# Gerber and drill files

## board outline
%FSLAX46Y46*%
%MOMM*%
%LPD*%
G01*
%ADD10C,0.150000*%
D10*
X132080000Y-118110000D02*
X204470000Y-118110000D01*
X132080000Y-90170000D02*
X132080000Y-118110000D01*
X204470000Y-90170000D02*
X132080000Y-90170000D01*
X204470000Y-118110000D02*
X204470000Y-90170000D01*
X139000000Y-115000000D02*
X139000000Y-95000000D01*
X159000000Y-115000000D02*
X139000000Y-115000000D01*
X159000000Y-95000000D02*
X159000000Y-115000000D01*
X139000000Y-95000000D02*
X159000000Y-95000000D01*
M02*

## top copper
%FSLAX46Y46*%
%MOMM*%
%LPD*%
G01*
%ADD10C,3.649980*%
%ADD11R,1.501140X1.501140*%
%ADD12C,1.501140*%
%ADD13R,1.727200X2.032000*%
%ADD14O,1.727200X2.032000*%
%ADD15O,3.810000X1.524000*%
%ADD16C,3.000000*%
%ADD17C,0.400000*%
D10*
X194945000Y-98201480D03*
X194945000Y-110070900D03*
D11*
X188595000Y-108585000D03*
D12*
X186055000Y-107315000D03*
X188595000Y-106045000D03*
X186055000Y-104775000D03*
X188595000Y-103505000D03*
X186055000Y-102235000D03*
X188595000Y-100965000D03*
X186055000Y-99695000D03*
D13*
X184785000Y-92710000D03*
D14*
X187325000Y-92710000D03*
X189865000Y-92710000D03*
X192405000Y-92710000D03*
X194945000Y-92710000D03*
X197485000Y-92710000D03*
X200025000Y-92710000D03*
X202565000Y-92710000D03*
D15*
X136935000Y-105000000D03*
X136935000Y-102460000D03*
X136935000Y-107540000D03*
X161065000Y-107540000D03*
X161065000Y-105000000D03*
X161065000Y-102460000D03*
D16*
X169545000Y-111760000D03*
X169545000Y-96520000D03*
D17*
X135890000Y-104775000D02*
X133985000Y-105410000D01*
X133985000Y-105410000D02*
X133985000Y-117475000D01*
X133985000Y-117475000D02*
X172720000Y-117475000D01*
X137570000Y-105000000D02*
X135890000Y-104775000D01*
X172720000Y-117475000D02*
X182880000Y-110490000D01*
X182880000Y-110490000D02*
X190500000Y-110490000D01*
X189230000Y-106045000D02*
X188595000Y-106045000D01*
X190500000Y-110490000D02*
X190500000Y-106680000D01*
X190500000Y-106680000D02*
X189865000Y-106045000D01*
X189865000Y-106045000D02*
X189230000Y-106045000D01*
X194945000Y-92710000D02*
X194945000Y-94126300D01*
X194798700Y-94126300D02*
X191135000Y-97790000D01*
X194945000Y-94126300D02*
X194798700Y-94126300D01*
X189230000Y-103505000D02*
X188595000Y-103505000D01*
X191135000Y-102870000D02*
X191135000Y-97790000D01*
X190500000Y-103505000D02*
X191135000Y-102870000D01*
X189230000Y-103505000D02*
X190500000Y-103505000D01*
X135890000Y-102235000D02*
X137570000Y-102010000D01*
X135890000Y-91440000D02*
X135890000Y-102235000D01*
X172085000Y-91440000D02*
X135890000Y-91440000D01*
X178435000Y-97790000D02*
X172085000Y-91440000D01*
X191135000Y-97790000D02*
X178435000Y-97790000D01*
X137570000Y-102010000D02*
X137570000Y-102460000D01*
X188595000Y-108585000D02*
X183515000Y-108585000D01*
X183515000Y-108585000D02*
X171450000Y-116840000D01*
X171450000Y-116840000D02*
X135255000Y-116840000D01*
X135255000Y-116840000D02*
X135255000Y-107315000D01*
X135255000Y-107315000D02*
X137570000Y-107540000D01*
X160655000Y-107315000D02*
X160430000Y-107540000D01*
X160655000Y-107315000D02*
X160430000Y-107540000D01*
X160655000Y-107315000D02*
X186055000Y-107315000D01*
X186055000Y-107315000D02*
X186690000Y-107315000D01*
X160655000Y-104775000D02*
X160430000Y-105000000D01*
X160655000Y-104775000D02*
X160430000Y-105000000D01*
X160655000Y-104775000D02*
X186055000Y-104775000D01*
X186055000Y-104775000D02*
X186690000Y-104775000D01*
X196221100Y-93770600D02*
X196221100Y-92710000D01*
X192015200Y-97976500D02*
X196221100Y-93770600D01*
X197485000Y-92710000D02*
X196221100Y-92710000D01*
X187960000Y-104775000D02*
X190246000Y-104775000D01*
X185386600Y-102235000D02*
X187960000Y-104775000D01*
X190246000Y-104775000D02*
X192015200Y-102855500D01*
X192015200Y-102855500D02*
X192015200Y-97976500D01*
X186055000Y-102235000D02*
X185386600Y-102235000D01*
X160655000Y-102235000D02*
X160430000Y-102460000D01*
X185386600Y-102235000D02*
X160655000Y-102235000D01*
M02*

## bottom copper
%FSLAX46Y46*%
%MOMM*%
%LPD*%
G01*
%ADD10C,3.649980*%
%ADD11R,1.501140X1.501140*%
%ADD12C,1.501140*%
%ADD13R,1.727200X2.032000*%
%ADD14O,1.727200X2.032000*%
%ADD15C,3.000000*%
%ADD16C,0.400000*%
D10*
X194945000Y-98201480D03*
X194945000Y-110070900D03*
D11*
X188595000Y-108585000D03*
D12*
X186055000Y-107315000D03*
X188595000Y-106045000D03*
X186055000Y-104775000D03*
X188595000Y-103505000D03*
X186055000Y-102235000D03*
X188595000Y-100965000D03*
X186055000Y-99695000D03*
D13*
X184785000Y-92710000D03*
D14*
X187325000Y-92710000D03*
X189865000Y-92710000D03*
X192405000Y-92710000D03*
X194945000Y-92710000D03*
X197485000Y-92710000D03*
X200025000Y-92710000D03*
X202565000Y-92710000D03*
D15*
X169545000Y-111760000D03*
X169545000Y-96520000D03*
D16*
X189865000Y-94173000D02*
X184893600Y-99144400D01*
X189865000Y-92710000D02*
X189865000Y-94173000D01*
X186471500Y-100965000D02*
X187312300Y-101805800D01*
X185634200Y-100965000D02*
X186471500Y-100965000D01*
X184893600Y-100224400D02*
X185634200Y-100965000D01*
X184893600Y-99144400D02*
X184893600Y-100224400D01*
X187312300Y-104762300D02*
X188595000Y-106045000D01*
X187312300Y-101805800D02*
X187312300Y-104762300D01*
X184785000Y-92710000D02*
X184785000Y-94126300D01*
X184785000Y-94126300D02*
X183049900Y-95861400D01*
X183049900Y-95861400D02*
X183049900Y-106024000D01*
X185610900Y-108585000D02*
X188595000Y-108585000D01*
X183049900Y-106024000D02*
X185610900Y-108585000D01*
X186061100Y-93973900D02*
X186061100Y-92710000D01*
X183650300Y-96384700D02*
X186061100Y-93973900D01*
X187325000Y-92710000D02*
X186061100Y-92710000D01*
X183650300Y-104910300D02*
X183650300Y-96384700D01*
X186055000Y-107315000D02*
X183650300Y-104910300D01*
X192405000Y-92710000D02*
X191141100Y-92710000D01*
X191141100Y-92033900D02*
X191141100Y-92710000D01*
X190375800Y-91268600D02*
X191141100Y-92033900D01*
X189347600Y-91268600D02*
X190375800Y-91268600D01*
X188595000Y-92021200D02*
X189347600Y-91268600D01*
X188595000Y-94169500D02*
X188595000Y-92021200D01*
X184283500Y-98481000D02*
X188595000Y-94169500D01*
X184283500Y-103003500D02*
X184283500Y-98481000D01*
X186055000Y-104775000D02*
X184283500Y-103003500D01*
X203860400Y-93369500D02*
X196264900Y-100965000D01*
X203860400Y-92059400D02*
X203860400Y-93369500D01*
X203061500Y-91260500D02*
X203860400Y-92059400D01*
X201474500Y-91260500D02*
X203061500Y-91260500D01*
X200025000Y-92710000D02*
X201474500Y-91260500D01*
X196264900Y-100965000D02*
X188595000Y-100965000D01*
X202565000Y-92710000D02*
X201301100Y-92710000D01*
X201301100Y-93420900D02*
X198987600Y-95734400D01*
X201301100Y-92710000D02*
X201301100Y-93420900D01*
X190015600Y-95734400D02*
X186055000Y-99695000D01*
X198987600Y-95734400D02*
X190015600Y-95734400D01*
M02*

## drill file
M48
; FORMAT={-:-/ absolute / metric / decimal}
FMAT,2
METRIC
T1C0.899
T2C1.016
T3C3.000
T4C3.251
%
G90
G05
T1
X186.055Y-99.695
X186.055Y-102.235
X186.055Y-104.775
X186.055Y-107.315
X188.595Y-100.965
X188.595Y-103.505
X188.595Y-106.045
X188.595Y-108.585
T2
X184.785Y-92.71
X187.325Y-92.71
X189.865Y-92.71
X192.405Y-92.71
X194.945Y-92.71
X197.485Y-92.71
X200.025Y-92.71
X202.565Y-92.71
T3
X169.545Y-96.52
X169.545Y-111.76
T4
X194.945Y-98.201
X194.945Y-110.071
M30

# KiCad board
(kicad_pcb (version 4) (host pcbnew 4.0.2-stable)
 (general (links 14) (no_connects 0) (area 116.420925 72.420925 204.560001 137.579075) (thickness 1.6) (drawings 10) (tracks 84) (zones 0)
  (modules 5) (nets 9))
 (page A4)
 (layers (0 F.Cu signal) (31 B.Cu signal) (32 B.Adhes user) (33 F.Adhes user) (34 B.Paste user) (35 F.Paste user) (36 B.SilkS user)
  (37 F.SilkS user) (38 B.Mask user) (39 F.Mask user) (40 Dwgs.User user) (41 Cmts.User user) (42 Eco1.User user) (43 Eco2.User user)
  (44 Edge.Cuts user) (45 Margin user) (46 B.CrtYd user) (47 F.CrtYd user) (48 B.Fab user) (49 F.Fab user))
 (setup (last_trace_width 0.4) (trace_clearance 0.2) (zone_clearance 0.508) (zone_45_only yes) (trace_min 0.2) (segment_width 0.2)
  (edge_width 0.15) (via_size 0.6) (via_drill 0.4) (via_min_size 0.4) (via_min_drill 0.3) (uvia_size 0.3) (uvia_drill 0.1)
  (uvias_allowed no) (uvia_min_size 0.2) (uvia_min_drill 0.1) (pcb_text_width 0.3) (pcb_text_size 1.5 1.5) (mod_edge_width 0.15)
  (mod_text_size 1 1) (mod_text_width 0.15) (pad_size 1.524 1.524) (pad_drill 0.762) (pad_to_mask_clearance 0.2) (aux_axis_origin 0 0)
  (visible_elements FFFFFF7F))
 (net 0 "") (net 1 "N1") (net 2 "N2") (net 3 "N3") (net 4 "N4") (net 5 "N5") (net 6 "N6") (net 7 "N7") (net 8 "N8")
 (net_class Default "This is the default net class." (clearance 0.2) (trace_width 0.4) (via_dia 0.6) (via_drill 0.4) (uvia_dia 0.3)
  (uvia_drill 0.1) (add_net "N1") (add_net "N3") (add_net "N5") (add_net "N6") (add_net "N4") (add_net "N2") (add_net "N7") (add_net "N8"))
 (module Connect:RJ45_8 (layer F.Cu) (at 194.945 104.14 90)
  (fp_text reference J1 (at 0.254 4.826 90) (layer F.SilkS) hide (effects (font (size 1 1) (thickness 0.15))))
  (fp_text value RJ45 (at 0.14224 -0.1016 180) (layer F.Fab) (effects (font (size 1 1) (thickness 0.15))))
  (pad Hole np_thru_hole circle (at 5.93852 0 90) (size 3.64998 3.64998) (drill 3.2512) (layers *.Cu *.SilkS *.Mask))
  (pad Hole np_thru_hole circle (at -5.9309 0 90) (size 3.64998 3.64998) (drill 3.2512) (layers *.Cu *.SilkS *.Mask))
  (pad 1 thru_hole rect (at -4.445 -6.35 90) (size 1.50114 1.50114) (drill 0.89916) (layers *.Cu *.Mask F.SilkS) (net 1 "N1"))
  (pad 2 thru_hole circle (at -3.175 -8.89 90) (size 1.50114 1.50114) (drill 0.89916) (layers *.Cu *.Mask F.SilkS) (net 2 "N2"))
  (pad 3 thru_hole circle (at -1.905 -6.35 90) (size 1.50114 1.50114) (drill 0.89916) (layers *.Cu *.Mask F.SilkS) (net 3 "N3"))
  (pad 4 thru_hole circle (at -0.635 -8.89 90) (size 1.50114 1.50114) (drill 0.89916) (layers *.Cu *.Mask F.SilkS) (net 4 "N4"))
  (pad 5 thru_hole circle (at 0.635 -6.35 90) (size 1.50114 1.50114) (drill 0.89916) (layers *.Cu *.Mask F.SilkS) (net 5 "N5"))
  (pad 6 thru_hole circle (at 1.905 -8.89 90) (size 1.50114 1.50114) (drill 0.89916) (layers *.Cu *.Mask F.SilkS) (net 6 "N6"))
  (pad 7 thru_hole circle (at 3.175 -6.35 90) (size 1.50114 1.50114) (drill 0.89916) (layers *.Cu *.Mask F.SilkS) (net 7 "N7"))
  (pad 8 thru_hole circle (at 4.445 -8.89 90) (size 1.50114 1.50114) (drill 0.89916) (layers *.Cu *.Mask F.SilkS) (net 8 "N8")))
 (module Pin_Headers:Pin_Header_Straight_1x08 (layer F.Cu) (at 184.785 92.71 90)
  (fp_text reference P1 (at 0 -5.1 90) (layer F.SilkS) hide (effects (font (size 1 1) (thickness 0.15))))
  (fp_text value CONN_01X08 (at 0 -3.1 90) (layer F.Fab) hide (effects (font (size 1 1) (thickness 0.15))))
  (pad 1 thru_hole rect (at 0 0 90) (size 2.032 1.7272) (drill 1.016) (layers *.Cu *.Mask F.SilkS) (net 1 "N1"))
  (pad 2 thru_hole oval (at 0 2.54 90) (size 2.032 1.7272) (drill 1.016) (layers *.Cu *.Mask F.SilkS) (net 2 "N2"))
  (pad 3 thru_hole oval (at 0 5.08 90) (size 2.032 1.7272) (drill 1.016) (layers *.Cu *.Mask F.SilkS) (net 3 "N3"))
  (pad 4 thru_hole oval (at 0 7.62 90) (size 2.032 1.7272) (drill 1.016) (layers *.Cu *.Mask F.SilkS) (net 4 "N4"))
  (pad 5 thru_hole oval (at 0 10.16 90) (size 2.032 1.7272) (drill 1.016) (layers *.Cu *.Mask F.SilkS) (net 5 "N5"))
  (pad 6 thru_hole oval (at 0 12.7 90) (size 2.032 1.7272) (drill 1.016) (layers *.Cu *.Mask F.SilkS) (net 6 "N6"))
  (pad 7 thru_hole oval (at 0 15.24 90) (size 2.032 1.7272) (drill 1.016) (layers *.Cu *.Mask F.SilkS) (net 7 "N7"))
  (pad 8 thru_hole oval (at 0 17.78 90) (size 2.032 1.7272) (drill 1.016) (layers *.Cu *.Mask F.SilkS) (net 8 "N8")))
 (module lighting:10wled (layer F.Cu) (at 149 105)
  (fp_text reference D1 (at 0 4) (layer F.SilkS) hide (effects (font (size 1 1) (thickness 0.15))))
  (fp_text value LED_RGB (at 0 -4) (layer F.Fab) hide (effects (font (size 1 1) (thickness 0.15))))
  (pad 2 smd oval (at -12.065 0) (size 3.81 1.524) (layers F.Cu F.Paste F.Mask) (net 3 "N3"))
  (pad 3 smd oval (at -12.065 -2.54) (size 3.81 1.524) (layers F.Cu F.Paste F.Mask) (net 5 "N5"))
  (pad 1 smd oval (at -12.065 2.54) (size 3.81 1.524) (layers F.Cu F.Paste F.Mask) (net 1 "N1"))
  (pad 6 smd oval (at 12.065 2.54) (size 3.81 1.524) (layers F.Cu F.Paste F.Mask) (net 2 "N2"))
  (pad 5 smd oval (at 12.065 0) (size 3.81 1.524) (layers F.Cu F.Paste F.Mask) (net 4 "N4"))
  (pad 4 smd oval (at 12.065 -2.54) (size 3.81 1.524) (layers F.Cu F.Paste F.Mask) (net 6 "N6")))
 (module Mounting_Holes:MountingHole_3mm (layer F.Cu) (at 169.545 111.76)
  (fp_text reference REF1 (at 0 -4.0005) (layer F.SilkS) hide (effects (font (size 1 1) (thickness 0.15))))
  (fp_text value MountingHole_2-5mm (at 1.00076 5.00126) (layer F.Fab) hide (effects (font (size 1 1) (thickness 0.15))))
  (pad 1 thru_hole circle (at 0 0) (size 3 3) (drill 3) (layers)))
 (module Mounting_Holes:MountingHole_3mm (layer F.Cu) (at 169.545 96.52)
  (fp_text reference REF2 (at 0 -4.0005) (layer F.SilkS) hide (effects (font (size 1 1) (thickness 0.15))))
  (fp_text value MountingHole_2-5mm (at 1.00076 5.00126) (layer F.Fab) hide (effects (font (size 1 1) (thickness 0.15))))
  (pad 1 thru_hole circle (at 0 0) (size 3 3) (drill 3) (layers)))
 (gr_line (start 132.08 118.11) (end 204.47 118.11) (angle 90) (layer Edge.Cuts) (width 0.15))
 (gr_line (start 132.08 90.17) (end 132.08 118.11) (angle 90) (layer Edge.Cuts) (width 0.15))
 (gr_line (start 204.47 90.17) (end 132.08 90.17) (angle 90) (layer Edge.Cuts) (width 0.15))
 (gr_line (start 204.47 118.11) (end 204.47 90.17) (angle 90) (layer Edge.Cuts) (width 0.15))
 (gr_line (start 139 115) (end 139 95) (angle 90) (layer Edge.Cuts) (width 0.15))
 (gr_line (start 159 115) (end 139 115) (angle 90) (layer Edge.Cuts) (width 0.15))
 (gr_line (start 159 95) (end 159 115) (angle 90) (layer Edge.Cuts) (width 0.15))
 (gr_line (start 139 95) (end 159 95) (angle 90) (layer Edge.Cuts) (width 0.15))
 (segment (start 189.865 94.173) (end 184.8936 99.1444) (width 0.4) (layer B.Cu) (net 3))
 (segment (start 189.865 92.71) (end 189.865 94.173) (width 0.4) (layer B.Cu) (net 3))
 (segment (start 186.4715 100.965) (end 187.3123 101.8058) (width 0.4) (layer B.Cu) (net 3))
 (segment (start 185.6342 100.965) (end 186.4715 100.965) (width 0.4) (layer B.Cu) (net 3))
 (segment (start 184.8936 100.2244) (end 185.6342 100.965) (width 0.4) (layer B.Cu) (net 3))
 (segment (start 184.8936 99.1444) (end 184.8936 100.2244) (width 0.4) (layer B.Cu) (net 3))
 (segment (start 187.3123 104.7623) (end 188.595 106.045) (width 0.4) (layer B.Cu) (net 3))
 (segment (start 187.3123 101.8058) (end 187.3123 104.7623) (width 0.4) (layer B.Cu) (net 3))
 (segment (start 135.89 104.775) (end 133.985 105.41) (width 0.4) (layer F.Cu) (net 3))
 (segment (start 133.985 105.41) (end 133.985 117.475) (width 0.4) (layer F.Cu) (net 3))
 (segment (start 133.985 117.475) (end 172.72 117.475) (width 0.4) (layer F.Cu) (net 3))
 (segment (start 137.57 105) (end 135.89 104.775) (width 0.4) (layer F.Cu) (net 3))
 (segment (start 172.72 117.475) (end 182.88 110.49) (width 0.4) (layer F.Cu) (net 3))
 (segment (start 182.88 110.49) (end 190.5 110.49) (width 0.4) (layer F.Cu) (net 3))
 (segment (start 189.23 106.045) (end 188.595 106.045) (width 0.4) (layer F.Cu) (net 3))
 (segment (start 190.5 110.49) (end 190.5 106.68) (width 0.4) (layer F.Cu) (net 3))
 (segment (start 190.5 106.68) (end 189.865 106.045) (width 0.4) (layer F.Cu) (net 3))
 (segment (start 189.865 106.045) (end 189.23 106.045) (width 0.4) (layer F.Cu) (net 3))
 (segment (start 194.945 92.71) (end 194.945 94.1263) (width 0.4) (layer F.Cu) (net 5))
 (segment (start 194.7987 94.1263) (end 191.135 97.79) (width 0.4) (layer F.Cu) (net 5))
 (segment (start 194.945 94.1263) (end 194.7987 94.1263) (width 0.4) (layer F.Cu) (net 5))
 (segment (start 189.23 103.505) (end 188.595 103.505) (width 0.4) (layer F.Cu) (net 5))
 (segment (start 191.135 102.87) (end 191.135 97.79) (width 0.4) (layer F.Cu) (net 5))
 (segment (start 190.5 103.505) (end 191.135 102.87) (width 0.4) (layer F.Cu) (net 5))
 (segment (start 189.23 103.505) (end 190.5 103.505) (width 0.4) (layer F.Cu) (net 5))
 (segment (start 135.89 102.235) (end 137.57 102.01) (width 0.4) (layer F.Cu) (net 5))
 (segment (start 135.89 91.44) (end 135.89 102.235) (width 0.4) (layer F.Cu) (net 5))
 (segment (start 172.085 91.44) (end 135.89 91.44) (width 0.4) (layer F.Cu) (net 5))
 (segment (start 178.435 97.79) (end 172.085 91.44) (width 0.4) (layer F.Cu) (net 5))
 (segment (start 191.135 97.79) (end 178.435 97.79) (width 0.4) (layer F.Cu) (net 5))
 (segment (start 137.57 102.01) (end 137.57 102.46) (width 0.4) (layer F.Cu) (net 5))
 (segment (start 184.785 92.71) (end 184.785 94.1263) (width 0.4) (layer B.Cu) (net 1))
 (segment (start 184.785 94.1263) (end 183.0499 95.8614) (width 0.4) (layer B.Cu) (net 1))
 (segment (start 183.0499 95.8614) (end 183.0499 106.024) (width 0.4) (layer B.Cu) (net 1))
 (segment (start 185.6109 108.585) (end 188.595 108.585) (width 0.4) (layer B.Cu) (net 1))
 (segment (start 183.0499 106.024) (end 185.6109 108.585) (width 0.4) (layer B.Cu) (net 1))
 (segment (start 188.595 108.585) (end 183.515 108.585) (width 0.4) (layer F.Cu) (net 1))
 (segment (start 183.515 108.585) (end 171.45 116.84) (width 0.4) (layer F.Cu) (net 1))
 (segment (start 171.45 116.84) (end 135.255 116.84) (width 0.4) (layer F.Cu) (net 1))
 (segment (start 135.255 116.84) (end 135.255 107.315) (width 0.4) (layer F.Cu) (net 1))
 (segment (start 135.255 107.315) (end 137.57 107.54) (width 0.4) (layer F.Cu) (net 1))
 (segment (start 186.0611 93.9739) (end 186.0611 92.71) (width 0.4) (layer B.Cu) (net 2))
 (segment (start 183.6503 96.3847) (end 186.0611 93.9739) (width 0.4) (layer B.Cu) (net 2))
 (segment (start 187.325 92.71) (end 186.0611 92.71) (width 0.4) (layer B.Cu) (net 2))
 (segment (start 183.6503 104.9103) (end 183.6503 96.3847) (width 0.4) (layer B.Cu) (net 2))
 (segment (start 186.055 107.315) (end 183.6503 104.9103) (width 0.4) (layer B.Cu) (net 2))
 (segment (start 160.655 107.315) (end 160.43 107.54) (width 0.4) (layer F.Cu) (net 2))
 (segment (start 160.655 107.315) (end 160.43 107.54) (width 0.4) (layer F.Cu) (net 2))
 (segment (start 160.655 107.315) (end 186.055 107.315) (width 0.4) (layer F.Cu) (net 2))
 (segment (start 186.055 107.315) (end 186.69 107.315) (width 0.4) (layer F.Cu) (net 2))
 (segment (start 192.405 92.71) (end 191.1411 92.71) (width 0.4) (layer B.Cu) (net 4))
 (segment (start 191.1411 92.0339) (end 191.1411 92.71) (width 0.4) (layer B.Cu) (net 4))
 (segment (start 190.3758 91.2686) (end 191.1411 92.0339) (width 0.4) (layer B.Cu) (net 4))
 (segment (start 189.3476 91.2686) (end 190.3758 91.2686) (width 0.4) (layer B.Cu) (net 4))
 (segment (start 188.595 92.0212) (end 189.3476 91.2686) (width 0.4) (layer B.Cu) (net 4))
 (segment (start 188.595 94.1695) (end 188.595 92.0212) (width 0.4) (layer B.Cu) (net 4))
 (segment (start 184.2835 98.481) (end 188.595 94.1695) (width 0.4) (layer B.Cu) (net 4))
 (segment (start 184.2835 103.0035) (end 184.2835 98.481) (width 0.4) (layer B.Cu) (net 4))
 (segment (start 186.055 104.775) (end 184.2835 103.0035) (width 0.4) (layer B.Cu) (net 4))
 (segment (start 160.655 104.775) (end 160.43 105) (width 0.4) (layer F.Cu) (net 4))
 (segment (start 160.655 104.775) (end 160.43 105) (width 0.4) (layer F.Cu) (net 4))
 (segment (start 160.655 104.775) (end 186.055 104.775) (width 0.4) (layer F.Cu) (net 4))
 (segment (start 186.055 104.775) (end 186.69 104.775) (width 0.4) (layer F.Cu) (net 4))
 (segment (start 196.2211 93.7706) (end 196.2211 92.71) (width 0.4) (layer F.Cu) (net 6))
 (segment (start 192.0152 97.9765) (end 196.2211 93.7706) (width 0.4) (layer F.Cu) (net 6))
 (segment (start 197.485 92.71) (end 196.2211 92.71) (width 0.4) (layer F.Cu) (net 6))
 (segment (start 187.96 104.775) (end 190.246 104.775) (width 0.4) (layer F.Cu) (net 6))
 (segment (start 185.3866 102.235) (end 187.96 104.775) (width 0.4) (layer F.Cu) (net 6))
 (segment (start 190.246 104.775) (end 192.0152 102.8555) (width 0.4) (layer F.Cu) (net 6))
 (segment (start 192.0152 102.8555) (end 192.0152 97.9765) (width 0.4) (layer F.Cu) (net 6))
 (segment (start 186.055 102.235) (end 185.3866 102.235) (width 0.4) (layer F.Cu) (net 6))
 (segment (start 160.655 102.235) (end 160.43 102.46) (width 0.4) (layer F.Cu) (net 6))
 (segment (start 185.3866 102.235) (end 160.655 102.235) (width 0.4) (layer F.Cu) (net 6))
 (segment (start 203.8604 93.3695) (end 196.2649 100.965) (width 0.4) (layer B.Cu) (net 7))
 (segment (start 203.8604 92.0594) (end 203.8604 93.3695) (width 0.4) (layer B.Cu) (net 7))
 (segment (start 203.0615 91.2605) (end 203.8604 92.0594) (width 0.4) (layer B.Cu) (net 7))
 (segment (start 201.4745 91.2605) (end 203.0615 91.2605) (width 0.4) (layer B.Cu) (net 7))
 (segment (start 200.025 92.71) (end 201.4745 91.2605) (width 0.4) (layer B.Cu) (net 7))
 (segment (start 196.2649 100.965) (end 188.595 100.965) (width 0.4) (layer B.Cu) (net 7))
 (segment (start 202.565 92.71) (end 201.3011 92.71) (width 0.4) (layer B.Cu) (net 8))
 (segment (start 201.3011 93.4209) (end 198.9876 95.7344) (width 0.4) (layer B.Cu) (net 8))
 (segment (start 201.3011 92.71) (end 201.3011 93.4209) (width 0.4) (layer B.Cu) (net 8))
 (segment (start 190.0156 95.7344) (end 186.055 99.695) (width 0.4) (layer B.Cu) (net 8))
 (segment (start 198.9876 95.7344) (end 190.0156 95.7344) (width 0.4) (layer B.Cu) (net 8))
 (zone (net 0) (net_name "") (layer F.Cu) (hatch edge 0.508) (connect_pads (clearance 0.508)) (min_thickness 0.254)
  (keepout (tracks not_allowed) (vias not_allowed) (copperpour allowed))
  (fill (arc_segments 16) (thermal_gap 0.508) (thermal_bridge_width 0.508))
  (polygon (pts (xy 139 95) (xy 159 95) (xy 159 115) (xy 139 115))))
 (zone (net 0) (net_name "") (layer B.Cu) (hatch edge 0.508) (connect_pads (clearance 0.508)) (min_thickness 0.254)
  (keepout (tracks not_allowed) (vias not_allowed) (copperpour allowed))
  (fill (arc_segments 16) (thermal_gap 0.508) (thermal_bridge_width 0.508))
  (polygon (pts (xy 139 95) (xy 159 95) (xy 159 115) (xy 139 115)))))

